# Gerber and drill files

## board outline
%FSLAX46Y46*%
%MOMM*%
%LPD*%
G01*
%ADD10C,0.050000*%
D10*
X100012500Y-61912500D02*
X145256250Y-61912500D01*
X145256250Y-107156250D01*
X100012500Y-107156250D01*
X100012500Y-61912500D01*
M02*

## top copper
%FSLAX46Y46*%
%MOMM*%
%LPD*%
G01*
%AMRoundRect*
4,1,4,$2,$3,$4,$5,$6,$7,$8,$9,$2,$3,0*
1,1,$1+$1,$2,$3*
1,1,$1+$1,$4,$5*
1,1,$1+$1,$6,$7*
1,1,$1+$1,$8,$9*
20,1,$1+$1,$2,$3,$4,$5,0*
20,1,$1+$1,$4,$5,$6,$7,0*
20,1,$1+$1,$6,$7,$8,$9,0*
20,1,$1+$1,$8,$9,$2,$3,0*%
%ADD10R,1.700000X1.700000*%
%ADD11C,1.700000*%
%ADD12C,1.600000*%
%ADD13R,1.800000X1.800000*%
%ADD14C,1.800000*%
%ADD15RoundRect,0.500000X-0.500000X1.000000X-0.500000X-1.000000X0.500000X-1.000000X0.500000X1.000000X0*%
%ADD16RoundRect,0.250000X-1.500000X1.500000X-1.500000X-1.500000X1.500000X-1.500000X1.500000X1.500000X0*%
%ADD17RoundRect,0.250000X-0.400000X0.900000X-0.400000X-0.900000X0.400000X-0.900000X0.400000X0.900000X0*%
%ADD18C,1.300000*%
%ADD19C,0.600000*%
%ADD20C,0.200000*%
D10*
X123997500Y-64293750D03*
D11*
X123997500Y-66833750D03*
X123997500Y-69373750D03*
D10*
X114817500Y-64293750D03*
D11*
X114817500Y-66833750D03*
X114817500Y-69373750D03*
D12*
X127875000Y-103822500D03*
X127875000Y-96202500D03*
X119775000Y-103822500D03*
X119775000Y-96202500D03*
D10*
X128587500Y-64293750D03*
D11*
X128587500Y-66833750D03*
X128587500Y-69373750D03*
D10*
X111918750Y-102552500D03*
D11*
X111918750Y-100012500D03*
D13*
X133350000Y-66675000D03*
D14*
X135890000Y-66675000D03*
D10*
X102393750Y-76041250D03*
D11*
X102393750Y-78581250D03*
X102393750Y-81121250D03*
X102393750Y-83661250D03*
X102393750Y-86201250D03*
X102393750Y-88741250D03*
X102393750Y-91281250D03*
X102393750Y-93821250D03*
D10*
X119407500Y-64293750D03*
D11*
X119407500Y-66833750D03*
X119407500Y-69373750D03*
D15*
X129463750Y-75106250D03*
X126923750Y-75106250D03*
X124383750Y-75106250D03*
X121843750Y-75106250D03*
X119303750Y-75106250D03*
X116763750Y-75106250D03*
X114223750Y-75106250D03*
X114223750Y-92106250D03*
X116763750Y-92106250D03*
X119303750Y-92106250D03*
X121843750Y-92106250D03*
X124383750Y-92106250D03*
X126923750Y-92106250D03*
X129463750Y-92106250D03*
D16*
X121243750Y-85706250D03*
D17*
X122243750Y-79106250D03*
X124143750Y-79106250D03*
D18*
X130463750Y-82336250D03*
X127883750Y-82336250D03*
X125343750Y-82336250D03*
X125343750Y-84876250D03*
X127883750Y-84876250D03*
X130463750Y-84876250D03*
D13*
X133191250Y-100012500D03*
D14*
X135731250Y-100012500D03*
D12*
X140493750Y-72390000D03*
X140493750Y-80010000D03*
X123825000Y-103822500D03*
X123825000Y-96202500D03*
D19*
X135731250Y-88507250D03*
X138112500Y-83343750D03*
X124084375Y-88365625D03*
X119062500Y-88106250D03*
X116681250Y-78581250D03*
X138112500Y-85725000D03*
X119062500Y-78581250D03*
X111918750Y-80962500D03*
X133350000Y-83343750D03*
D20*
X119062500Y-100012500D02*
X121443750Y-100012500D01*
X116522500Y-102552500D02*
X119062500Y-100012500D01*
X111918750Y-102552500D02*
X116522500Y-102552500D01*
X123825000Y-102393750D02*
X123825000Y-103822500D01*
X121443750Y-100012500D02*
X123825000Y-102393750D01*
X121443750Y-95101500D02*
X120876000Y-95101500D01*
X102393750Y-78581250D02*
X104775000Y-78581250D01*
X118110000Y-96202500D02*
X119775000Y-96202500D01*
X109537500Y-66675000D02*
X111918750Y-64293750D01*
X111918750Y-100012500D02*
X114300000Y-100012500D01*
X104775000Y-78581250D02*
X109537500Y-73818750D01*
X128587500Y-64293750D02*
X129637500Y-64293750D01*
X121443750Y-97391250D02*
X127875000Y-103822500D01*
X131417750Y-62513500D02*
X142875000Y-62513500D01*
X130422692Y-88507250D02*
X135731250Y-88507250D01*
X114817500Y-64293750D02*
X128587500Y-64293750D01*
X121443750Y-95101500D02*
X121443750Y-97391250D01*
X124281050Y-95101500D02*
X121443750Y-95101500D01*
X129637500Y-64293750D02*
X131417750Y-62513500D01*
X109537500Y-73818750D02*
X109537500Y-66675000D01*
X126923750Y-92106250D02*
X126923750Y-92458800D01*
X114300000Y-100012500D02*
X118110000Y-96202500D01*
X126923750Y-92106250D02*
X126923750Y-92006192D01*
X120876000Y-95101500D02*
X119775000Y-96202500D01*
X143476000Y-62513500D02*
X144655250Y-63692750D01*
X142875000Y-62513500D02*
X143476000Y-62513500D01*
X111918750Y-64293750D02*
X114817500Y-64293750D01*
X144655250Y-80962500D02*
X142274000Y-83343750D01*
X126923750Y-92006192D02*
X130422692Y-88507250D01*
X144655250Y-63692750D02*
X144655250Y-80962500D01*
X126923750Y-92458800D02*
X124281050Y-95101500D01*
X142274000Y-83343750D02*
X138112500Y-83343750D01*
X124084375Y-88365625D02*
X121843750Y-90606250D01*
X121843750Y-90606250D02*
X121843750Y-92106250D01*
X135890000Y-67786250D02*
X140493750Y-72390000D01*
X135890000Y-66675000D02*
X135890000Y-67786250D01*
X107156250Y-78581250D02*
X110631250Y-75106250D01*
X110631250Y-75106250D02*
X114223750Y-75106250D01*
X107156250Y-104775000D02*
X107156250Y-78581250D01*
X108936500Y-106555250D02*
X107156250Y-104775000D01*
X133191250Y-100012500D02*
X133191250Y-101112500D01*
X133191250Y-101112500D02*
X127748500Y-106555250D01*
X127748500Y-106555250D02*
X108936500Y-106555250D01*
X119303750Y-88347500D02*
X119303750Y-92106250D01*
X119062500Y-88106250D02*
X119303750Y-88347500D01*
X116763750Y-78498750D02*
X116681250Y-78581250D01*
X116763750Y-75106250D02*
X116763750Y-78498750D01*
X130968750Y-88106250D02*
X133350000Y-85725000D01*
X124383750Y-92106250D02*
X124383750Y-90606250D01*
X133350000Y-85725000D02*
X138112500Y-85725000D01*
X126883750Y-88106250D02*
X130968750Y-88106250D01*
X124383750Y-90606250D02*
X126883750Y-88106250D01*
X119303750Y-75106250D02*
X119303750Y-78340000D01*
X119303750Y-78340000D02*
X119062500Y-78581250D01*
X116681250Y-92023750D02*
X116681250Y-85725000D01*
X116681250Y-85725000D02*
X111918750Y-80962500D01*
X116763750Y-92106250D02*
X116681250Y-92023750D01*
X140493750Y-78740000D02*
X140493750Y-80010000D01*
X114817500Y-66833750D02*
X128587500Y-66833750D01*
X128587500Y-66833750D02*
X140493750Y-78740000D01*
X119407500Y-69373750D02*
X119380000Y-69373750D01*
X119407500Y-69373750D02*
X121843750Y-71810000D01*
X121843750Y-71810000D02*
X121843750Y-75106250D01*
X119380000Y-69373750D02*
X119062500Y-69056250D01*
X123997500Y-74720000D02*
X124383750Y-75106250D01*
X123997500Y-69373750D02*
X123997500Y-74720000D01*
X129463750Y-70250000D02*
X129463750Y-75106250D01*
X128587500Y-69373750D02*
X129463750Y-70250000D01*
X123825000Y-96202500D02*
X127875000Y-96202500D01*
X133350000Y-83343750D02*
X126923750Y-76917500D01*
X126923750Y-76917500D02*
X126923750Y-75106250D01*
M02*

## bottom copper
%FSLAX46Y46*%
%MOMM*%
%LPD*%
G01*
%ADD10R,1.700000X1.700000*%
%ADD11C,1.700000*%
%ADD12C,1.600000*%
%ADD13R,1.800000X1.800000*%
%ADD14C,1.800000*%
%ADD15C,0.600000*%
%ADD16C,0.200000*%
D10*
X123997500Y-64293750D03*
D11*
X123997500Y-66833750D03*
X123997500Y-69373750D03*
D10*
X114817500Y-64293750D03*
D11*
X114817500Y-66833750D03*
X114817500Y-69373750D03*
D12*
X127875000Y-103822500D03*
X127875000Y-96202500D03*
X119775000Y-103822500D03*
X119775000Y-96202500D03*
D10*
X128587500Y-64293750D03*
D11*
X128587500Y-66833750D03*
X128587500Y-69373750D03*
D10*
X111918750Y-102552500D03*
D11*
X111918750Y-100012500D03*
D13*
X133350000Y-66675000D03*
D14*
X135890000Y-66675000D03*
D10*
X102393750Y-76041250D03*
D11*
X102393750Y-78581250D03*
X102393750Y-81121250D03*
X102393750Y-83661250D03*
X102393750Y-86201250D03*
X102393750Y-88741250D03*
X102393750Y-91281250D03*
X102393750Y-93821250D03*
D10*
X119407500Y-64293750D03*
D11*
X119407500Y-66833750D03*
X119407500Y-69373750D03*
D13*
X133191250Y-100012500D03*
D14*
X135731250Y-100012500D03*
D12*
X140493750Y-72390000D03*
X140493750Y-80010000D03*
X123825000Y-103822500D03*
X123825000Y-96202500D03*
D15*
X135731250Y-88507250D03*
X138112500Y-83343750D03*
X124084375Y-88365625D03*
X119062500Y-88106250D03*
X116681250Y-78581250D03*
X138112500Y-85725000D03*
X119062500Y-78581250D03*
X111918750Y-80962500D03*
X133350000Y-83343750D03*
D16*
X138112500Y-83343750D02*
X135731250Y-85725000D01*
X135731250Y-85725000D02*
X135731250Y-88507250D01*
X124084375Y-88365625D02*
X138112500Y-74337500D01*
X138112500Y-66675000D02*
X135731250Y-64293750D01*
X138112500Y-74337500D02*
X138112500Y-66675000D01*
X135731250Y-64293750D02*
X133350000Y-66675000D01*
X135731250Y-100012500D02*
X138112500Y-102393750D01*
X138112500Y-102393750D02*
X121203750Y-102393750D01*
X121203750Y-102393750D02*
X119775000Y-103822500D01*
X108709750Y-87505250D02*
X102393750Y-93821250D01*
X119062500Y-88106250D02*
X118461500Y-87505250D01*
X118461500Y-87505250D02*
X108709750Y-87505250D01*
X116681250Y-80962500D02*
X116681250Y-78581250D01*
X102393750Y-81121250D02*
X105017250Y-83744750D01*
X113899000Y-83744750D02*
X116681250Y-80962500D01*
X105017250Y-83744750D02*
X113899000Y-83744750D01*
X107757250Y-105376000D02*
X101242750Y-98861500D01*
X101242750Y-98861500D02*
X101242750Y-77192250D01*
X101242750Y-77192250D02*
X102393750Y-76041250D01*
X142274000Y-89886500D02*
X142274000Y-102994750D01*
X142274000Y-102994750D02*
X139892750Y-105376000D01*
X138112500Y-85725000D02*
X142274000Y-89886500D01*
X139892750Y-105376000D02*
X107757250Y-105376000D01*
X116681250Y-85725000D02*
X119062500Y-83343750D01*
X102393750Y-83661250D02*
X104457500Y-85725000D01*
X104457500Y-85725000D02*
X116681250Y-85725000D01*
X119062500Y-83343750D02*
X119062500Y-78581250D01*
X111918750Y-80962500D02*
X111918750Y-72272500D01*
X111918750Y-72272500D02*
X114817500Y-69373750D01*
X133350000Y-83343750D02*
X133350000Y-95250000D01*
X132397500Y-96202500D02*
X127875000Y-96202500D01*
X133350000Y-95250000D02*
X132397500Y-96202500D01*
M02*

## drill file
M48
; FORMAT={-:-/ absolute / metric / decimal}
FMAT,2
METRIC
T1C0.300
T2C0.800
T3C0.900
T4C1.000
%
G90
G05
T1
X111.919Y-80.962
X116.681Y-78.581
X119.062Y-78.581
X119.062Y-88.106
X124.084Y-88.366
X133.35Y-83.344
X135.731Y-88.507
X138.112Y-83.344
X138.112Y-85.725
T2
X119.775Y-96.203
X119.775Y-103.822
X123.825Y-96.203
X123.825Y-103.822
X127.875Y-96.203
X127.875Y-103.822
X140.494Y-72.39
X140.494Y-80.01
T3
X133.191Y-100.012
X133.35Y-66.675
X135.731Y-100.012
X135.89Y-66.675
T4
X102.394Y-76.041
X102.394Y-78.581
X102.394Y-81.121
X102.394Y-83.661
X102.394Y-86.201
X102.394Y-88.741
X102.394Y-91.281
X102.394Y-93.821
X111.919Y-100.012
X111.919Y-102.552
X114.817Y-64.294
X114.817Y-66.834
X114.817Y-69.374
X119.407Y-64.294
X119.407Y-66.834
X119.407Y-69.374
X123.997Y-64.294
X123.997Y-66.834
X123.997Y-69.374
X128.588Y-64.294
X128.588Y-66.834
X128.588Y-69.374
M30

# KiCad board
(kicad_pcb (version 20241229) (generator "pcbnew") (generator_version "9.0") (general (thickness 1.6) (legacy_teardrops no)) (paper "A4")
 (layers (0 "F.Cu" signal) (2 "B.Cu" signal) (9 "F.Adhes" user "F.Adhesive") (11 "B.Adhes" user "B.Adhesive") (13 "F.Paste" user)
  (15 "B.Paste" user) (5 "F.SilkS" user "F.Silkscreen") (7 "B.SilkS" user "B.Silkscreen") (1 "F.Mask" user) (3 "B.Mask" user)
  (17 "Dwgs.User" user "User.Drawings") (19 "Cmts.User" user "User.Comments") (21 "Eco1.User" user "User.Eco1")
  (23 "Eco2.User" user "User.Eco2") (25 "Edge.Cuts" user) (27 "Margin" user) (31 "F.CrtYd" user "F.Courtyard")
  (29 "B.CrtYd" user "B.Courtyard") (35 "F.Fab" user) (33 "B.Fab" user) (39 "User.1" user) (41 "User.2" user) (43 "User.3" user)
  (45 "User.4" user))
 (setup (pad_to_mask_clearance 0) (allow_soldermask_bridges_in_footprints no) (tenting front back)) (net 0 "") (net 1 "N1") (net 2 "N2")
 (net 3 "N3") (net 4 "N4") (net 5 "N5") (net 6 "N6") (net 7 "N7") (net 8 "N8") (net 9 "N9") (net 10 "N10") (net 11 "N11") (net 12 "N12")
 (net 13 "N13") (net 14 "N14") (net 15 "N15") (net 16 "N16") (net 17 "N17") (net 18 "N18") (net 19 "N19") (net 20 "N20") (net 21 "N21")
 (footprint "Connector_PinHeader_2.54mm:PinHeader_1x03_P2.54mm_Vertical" (layer "F.Cu") (at 123.9975 64.29375)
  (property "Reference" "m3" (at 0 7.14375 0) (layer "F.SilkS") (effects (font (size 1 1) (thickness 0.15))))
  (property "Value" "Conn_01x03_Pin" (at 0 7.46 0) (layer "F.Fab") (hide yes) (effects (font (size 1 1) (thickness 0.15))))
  (pad "1" thru_hole rect (at 0 0) (size 1.7 1.7) (drill 1) (layers "*.Cu" "*.Mask") (remove_unused_layers no) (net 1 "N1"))
  (pad "2" thru_hole circle (at 0 2.54) (size 1.7 1.7) (drill 1) (layers "*.Cu" "*.Mask") (remove_unused_layers no) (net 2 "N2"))
  (pad "3" thru_hole circle (at 0 5.08) (size 1.7 1.7) (drill 1) (layers "*.Cu" "*.Mask") (remove_unused_layers no) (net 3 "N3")))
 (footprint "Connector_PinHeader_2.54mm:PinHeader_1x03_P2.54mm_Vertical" (layer "F.Cu") (at 114.8175 64.29375)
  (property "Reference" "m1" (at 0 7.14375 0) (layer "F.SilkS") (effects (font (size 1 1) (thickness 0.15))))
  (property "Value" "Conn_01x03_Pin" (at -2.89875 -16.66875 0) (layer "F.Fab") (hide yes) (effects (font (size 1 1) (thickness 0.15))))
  (pad "1" thru_hole rect (at 0 0) (size 1.7 1.7) (drill 1) (layers "*.Cu" "*.Mask") (remove_unused_layers no) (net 1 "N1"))
  (pad "2" thru_hole circle (at 0 2.54) (size 1.7 1.7) (drill 1) (layers "*.Cu" "*.Mask") (remove_unused_layers no) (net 2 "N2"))
  (pad "3" thru_hole circle (at 0 5.08) (size 1.7 1.7) (drill 1) (layers "*.Cu" "*.Mask") (remove_unused_layers no) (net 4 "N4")))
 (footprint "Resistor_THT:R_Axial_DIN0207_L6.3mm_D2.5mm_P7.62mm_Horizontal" (layer "F.Cu") (at 127.875 103.8225 90)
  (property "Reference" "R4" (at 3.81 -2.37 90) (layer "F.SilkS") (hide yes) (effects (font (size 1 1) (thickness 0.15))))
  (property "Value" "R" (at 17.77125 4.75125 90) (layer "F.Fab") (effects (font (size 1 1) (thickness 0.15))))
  (pad "1" thru_hole circle (at 0 0 90) (size 1.6 1.6) (drill 0.8) (layers "*.Cu" "*.Mask") (remove_unused_layers no) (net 1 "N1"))
  (pad "2" thru_hole circle (at 7.62 0 90) (size 1.6 1.6) (drill 0.8) (layers "*.Cu" "*.Mask") (remove_unused_layers no) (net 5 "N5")))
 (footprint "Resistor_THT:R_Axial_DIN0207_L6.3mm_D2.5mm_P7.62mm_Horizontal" (layer "F.Cu") (at 119.775 103.8225 90)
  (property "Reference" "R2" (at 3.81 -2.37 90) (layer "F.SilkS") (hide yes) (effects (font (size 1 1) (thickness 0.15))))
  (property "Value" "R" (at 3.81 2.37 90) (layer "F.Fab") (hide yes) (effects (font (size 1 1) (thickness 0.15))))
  (pad "1" thru_hole circle (at 0 0 90) (size 1.6 1.6) (drill 0.8) (layers "*.Cu" "*.Mask") (remove_unused_layers no) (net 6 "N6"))
  (pad "2" thru_hole circle (at 7.62 0 90) (size 1.6 1.6) (drill 0.8) (layers "*.Cu" "*.Mask") (remove_unused_layers no) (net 1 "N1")))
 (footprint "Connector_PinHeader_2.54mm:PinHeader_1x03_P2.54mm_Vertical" (layer "F.Cu") (at 128.5875 64.29375)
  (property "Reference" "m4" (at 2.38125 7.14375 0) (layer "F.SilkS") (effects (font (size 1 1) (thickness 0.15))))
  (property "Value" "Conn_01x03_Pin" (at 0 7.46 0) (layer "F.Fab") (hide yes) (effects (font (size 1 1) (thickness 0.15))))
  (pad "1" thru_hole rect (at 0 0) (size 1.7 1.7) (drill 1) (layers "*.Cu" "*.Mask") (remove_unused_layers no) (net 1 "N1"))
  (pad "2" thru_hole circle (at 0 2.54) (size 1.7 1.7) (drill 1) (layers "*.Cu" "*.Mask") (remove_unused_layers no) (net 2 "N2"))
  (pad "3" thru_hole circle (at 0 5.08) (size 1.7 1.7) (drill 1) (layers "*.Cu" "*.Mask") (remove_unused_layers no) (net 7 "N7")))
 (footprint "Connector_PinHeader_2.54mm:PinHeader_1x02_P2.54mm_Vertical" (layer "F.Cu") (at 111.91875 102.5525 180)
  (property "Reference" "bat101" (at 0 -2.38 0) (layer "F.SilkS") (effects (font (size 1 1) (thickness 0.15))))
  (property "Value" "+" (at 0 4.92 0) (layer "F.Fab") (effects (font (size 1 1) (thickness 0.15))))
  (pad "1" thru_hole rect (at 0 0 180) (size 1.7 1.7) (drill 1) (layers "*.Cu" "*.Mask") (remove_unused_layers no) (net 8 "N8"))
  (pad "2" thru_hole circle (at 0 2.54 180) (size 1.7 1.7) (drill 1) (layers "*.Cu" "*.Mask") (remove_unused_layers no) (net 1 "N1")))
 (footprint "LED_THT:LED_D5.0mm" (layer "F.Cu") (at 133.35 66.675)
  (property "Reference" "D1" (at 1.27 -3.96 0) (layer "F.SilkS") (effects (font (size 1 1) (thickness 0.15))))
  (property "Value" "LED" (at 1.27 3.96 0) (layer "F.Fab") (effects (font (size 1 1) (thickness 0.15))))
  (pad "1" thru_hole rect (at 0 0) (size 1.8 1.8) (drill 0.9) (layers "*.Cu" "*.Mask") (remove_unused_layers no) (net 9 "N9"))
  (pad "2" thru_hole circle (at 2.54 0) (size 1.8 1.8) (drill 0.9) (layers "*.Cu" "*.Mask") (remove_unused_layers no) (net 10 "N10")))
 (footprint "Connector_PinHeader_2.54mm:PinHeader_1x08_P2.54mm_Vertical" (layer "F.Cu") (at 102.39375 76.04125)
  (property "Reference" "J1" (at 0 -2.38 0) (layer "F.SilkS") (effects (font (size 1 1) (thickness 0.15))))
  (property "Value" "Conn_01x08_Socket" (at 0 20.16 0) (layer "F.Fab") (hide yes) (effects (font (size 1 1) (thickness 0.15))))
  (pad "1" thru_hole rect (at 0 0) (size 1.7 1.7) (drill 1) (layers "*.Cu" "*.Mask") (remove_unused_layers no) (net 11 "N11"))
  (pad "2" thru_hole circle (at 0 2.54) (size 1.7 1.7) (drill 1) (layers "*.Cu" "*.Mask") (remove_unused_layers no) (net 1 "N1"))
  (pad "3" thru_hole circle (at 0 5.08) (size 1.7 1.7) (drill 1) (layers "*.Cu" "*.Mask") (remove_unused_layers no) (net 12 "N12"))
  (pad "4" thru_hole circle (at 0 7.62) (size 1.7 1.7) (drill 1) (layers "*.Cu" "*.Mask") (remove_unused_layers no) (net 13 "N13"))
  (pad "5" thru_hole circle (at 0 10.16) (size 1.7 1.7) (drill 1) (layers "*.Cu" "*.Mask") (remove_unused_layers no) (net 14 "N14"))
  (pad "6" thru_hole circle (at 0 12.7) (size 1.7 1.7) (drill 1) (layers "*.Cu" "*.Mask") (remove_unused_layers no) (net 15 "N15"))
  (pad "7" thru_hole circle (at 0 15.24) (size 1.7 1.7) (drill 1) (layers "*.Cu" "*.Mask") (remove_unused_layers no) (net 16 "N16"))
  (pad "8" thru_hole circle (at 0 17.78) (size 1.7 1.7) (drill 1) (layers "*.Cu" "*.Mask") (remove_unused_layers no) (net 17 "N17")))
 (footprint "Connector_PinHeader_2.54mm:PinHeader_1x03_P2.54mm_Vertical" (layer "F.Cu") (at 119.4075 64.29375)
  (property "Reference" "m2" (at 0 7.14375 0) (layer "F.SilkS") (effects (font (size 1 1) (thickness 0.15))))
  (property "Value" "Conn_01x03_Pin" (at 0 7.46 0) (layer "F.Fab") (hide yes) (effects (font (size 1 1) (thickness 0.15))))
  (pad "1" thru_hole rect (at 0 0) (size 1.7 1.7) (drill 1) (layers "*.Cu" "*.Mask") (remove_unused_layers no) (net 1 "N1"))
  (pad "2" thru_hole circle (at 0 2.54) (size 1.7 1.7) (drill 1) (layers "*.Cu" "*.Mask") (remove_unused_layers no) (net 2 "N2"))
  (pad "3" thru_hole circle (at 0 5.08) (size 1.7 1.7) (drill 1) (layers "*.Cu" "*.Mask") (remove_unused_layers no) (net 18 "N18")))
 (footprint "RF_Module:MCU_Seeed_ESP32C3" (layer "F.Cu") (at 121.84375 83.60625 -90)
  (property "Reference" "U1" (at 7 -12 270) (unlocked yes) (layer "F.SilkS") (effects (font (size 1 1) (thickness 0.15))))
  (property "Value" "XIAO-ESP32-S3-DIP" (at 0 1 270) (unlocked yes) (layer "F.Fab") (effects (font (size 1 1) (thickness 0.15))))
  (pad "" smd roundrect (at 1.1 -0.4 270) (size 1.5 1.5) (layers "F.Paste") (roundrect_rratio 0.1666666667))
  (pad "" smd roundrect (at 1.1 1.6 270) (size 1.5 1.5) (layers "F.Paste") (roundrect_rratio 0.1666666667))
  (pad "" smd roundrect (at 3.1 -0.4 270) (size 1.5 1.5) (layers "F.Paste") (roundrect_rratio 0.1666666667))
  (pad "" smd roundrect (at 3.1 1.6 270) (size 1.5 1.5) (layers "F.Paste") (roundrect_rratio 0.1666666667))
  (pad "1" smd roundrect (at -8.5 -7.62 270) (size 3 2) (layers "F.Cu" "F.Mask" "F.Paste") (roundrect_rratio 0.25) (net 7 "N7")
   (thermal_bridge_angle 45))
  (pad "2" smd roundrect (at -8.5 -5.08 270) (size 3 2) (layers "F.Cu" "F.Mask" "F.Paste") (roundrect_rratio 0.25) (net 5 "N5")
   (thermal_bridge_angle 45))
  (pad "3" smd roundrect (at -8.5 -2.54 270) (size 3 2) (layers "F.Cu" "F.Mask" "F.Paste") (roundrect_rratio 0.25) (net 3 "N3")
   (thermal_bridge_angle 45))
  (pad "4" smd roundrect (at -8.5 0 270) (size 3 2) (layers "F.Cu" "F.Mask" "F.Paste") (roundrect_rratio 0.25) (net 18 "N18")
   (thermal_bridge_angle 45))
  (pad "5" smd roundrect (at -8.5 2.54 270) (size 3 2) (layers "F.Cu" "F.Mask" "F.Paste") (roundrect_rratio 0.25) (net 13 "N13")
   (thermal_bridge_angle 45))
  (pad "6" smd roundrect (at -8.5 5.08 270) (size 3 2) (layers "F.Cu" "F.Mask" "F.Paste") (roundrect_rratio 0.25) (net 12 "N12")
   (thermal_bridge_angle 45))
  (pad "7" smd roundrect (at -8.5 7.62 270) (size 3 2) (layers "F.Cu" "F.Mask" "F.Paste") (roundrect_rratio 0.25) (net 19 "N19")
   (thermal_bridge_angle 45))
  (pad "8" smd roundrect (at 8.5 7.62 270) (size 3 2) (layers "F.Cu" "F.Mask" "F.Paste") (roundrect_rratio 0.25) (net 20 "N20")
   (thermal_bridge_angle 45))
  (pad "9" smd roundrect (at 8.5 5.08 270) (size 3 2) (layers "F.Cu" "F.Mask" "F.Paste") (roundrect_rratio 0.25) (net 4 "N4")
   (thermal_bridge_angle 45))
  (pad "10" smd roundrect (at 8.5 2.54 270) (size 3 2) (layers "F.Cu" "F.Mask" "F.Paste") (roundrect_rratio 0.25) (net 17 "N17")
   (thermal_bridge_angle 45))
  (pad "11" smd roundrect (at 8.5 0 270) (size 3 2) (layers "F.Cu" "F.Mask" "F.Paste") (roundrect_rratio 0.25) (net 9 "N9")
   (thermal_bridge_angle 45))
  (pad "12" smd roundrect (at 8.5 -2.54 270) (size 3 2) (layers "F.Cu" "F.Mask" "F.Paste") (roundrect_rratio 0.25) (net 11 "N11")
   (thermal_bridge_angle 45))
  (pad "13" smd roundrect (at 8.5 -5.08 270) (size 3 2) (layers "F.Cu" "F.Mask" "F.Paste") (roundrect_rratio 0.25) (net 1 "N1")
   (thermal_bridge_angle 45))
  (pad "14" smd roundrect (at 8.5 -7.62 270) (size 3 2) (layers "F.Cu" "F.Mask" "F.Paste") (roundrect_rratio 0.25) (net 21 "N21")
   (thermal_bridge_angle 45))
  (pad "15" smd roundrect (at 2.1 0.6 270) (size 3.5 3.5) (layers "F.Cu" "F.Mask") (roundrect_rratio 0.07142857143))
  (pad "16" smd roundrect (at -4.5 -0.4 270) (size 2.3 1.3) (layers "F.Cu" "F.Mask" "F.Paste") (roundrect_rratio 0.1923076923))
  (pad "17" smd roundrect (at -4.5 -2.3 270) (size 2.3 1.3) (layers "F.Cu" "F.Mask" "F.Paste") (roundrect_rratio 0.1923076923))
  (pad "18" smd circle (at -1.27 -8.62 270) (size 1.3 1.3) (layers "F.Cu" "F.Mask" "F.Paste"))
  (pad "19" smd circle (at -1.27 -6.04 270) (size 1.3 1.3) (layers "F.Cu" "F.Mask" "F.Paste"))
  (pad "20" smd circle (at -1.27 -3.5 270) (size 1.3 1.3) (layers "F.Cu" "F.Mask" "F.Paste"))
  (pad "21" smd circle (at 1.27 -3.5 270) (size 1.3 1.3) (layers "F.Cu" "F.Mask" "F.Paste"))
  (pad "22" smd circle (at 1.27 -6.04 270) (size 1.3 1.3) (layers "F.Cu" "F.Mask" "F.Paste"))
  (pad "23" smd circle (at 1.27 -8.62 270) (size 1.3 1.3) (layers "F.Cu" "F.Mask" "F.Paste")))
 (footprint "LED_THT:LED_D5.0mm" (layer "F.Cu") (at 133.19125 100.0125)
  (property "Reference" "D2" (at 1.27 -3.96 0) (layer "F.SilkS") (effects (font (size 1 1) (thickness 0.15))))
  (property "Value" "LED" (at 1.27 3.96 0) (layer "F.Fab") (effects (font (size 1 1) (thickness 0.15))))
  (pad "1" thru_hole rect (at 0 0) (size 1.8 1.8) (drill 0.9) (layers "*.Cu" "*.Mask") (remove_unused_layers no) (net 19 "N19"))
  (pad "2" thru_hole circle (at 2.54 0) (size 1.8 1.8) (drill 0.9) (layers "*.Cu" "*.Mask") (remove_unused_layers no) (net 6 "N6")))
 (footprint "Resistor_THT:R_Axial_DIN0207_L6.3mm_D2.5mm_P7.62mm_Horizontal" (layer "F.Cu") (at 140.49375 72.39 -90)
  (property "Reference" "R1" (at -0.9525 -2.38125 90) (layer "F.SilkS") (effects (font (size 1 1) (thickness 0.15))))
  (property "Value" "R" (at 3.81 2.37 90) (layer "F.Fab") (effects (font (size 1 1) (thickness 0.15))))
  (pad "1" thru_hole circle (at 0 0 270) (size 1.6 1.6) (drill 0.8) (layers "*.Cu" "*.Mask") (remove_unused_layers no) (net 10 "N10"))
  (pad "2" thru_hole circle (at 7.62 0 270) (size 1.6 1.6) (drill 0.8) (layers "*.Cu" "*.Mask") (remove_unused_layers no) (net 2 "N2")))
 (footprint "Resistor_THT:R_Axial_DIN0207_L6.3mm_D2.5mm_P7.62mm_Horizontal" (layer "F.Cu") (at 123.825 103.8225 90)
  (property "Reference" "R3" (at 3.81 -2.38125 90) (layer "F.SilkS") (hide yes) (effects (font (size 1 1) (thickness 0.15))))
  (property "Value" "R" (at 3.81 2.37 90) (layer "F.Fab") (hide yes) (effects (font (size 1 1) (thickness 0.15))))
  (pad "1" thru_hole circle (at 0 0 90) (size 1.6 1.6) (drill 0.8) (layers "*.Cu" "*.Mask") (remove_unused_layers no) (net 8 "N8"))
  (pad "2" thru_hole circle (at 7.62 0 90) (size 1.6 1.6) (drill 0.8) (layers "*.Cu" "*.Mask") (remove_unused_layers no) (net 5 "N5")))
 (gr_rect (start 100.0125 61.9125) (end 145.25625 107.15625) (stroke (width 0.05) (type default)) (fill no) (layer "Edge.Cuts"))
 (segment (start 119.0625 100.0125) (end 121.44375 100.0125) (width 0.2) (layer "F.Cu") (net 8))
 (segment (start 116.5225 102.5525) (end 119.0625 100.0125) (width 0.2) (layer "F.Cu") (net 8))
 (segment (start 111.91875 102.5525) (end 116.5225 102.5525) (width 0.2) (layer "F.Cu") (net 8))
 (segment (start 123.825 102.39375) (end 123.825 103.8225) (width 0.2) (layer "F.Cu") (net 8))
 (segment (start 121.44375 100.0125) (end 123.825 102.39375) (width 0.2) (layer "F.Cu") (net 8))
 (segment (start 121.44375 95.1015) (end 120.876 95.1015) (width 0.2) (layer "F.Cu") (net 1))
 (segment (start 102.39375 78.58125) (end 104.775 78.58125) (width 0.2) (layer "F.Cu") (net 1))
 (segment (start 118.11 96.2025) (end 119.775 96.2025) (width 0.2) (layer "F.Cu") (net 1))
 (segment (start 109.5375 66.675) (end 111.91875 64.29375) (width 0.2) (layer "F.Cu") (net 1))
 (segment (start 111.91875 100.0125) (end 114.3 100.0125) (width 0.2) (layer "F.Cu") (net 1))
 (segment (start 104.775 78.58125) (end 109.5375 73.81875) (width 0.2) (layer "F.Cu") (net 1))
 (segment (start 128.5875 64.29375) (end 129.6375 64.29375) (width 0.2) (layer "F.Cu") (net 1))
 (segment (start 121.44375 97.39125) (end 127.875 103.8225) (width 0.2) (layer "F.Cu") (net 1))
 (segment (start 131.41775 62.5135) (end 142.875 62.5135) (width 0.2) (layer "F.Cu") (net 1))
 (segment (start 130.422692 88.50725) (end 135.73125 88.50725) (width 0.2) (layer "F.Cu") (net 1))
 (segment (start 114.8175 64.29375) (end 128.5875 64.29375) (width 0.2) (layer "F.Cu") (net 1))
 (segment (start 121.44375 95.1015) (end 121.44375 97.39125) (width 0.2) (layer "F.Cu") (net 1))
 (segment (start 124.28105 95.1015) (end 121.44375 95.1015) (width 0.2) (layer "F.Cu") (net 1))
 (segment (start 129.6375 64.29375) (end 131.41775 62.5135) (width 0.2) (layer "F.Cu") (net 1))
 (segment (start 109.5375 73.81875) (end 109.5375 66.675) (width 0.2) (layer "F.Cu") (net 1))
 (segment (start 126.92375 92.10625) (end 126.92375 92.4588) (width 0.2) (layer "F.Cu") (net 1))
 (segment (start 114.3 100.0125) (end 118.11 96.2025) (width 0.2) (layer "F.Cu") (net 1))
 (segment (start 126.92375 92.10625) (end 126.92375 92.006192) (width 0.2) (layer "F.Cu") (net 1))
 (segment (start 120.876 95.1015) (end 119.775 96.2025) (width 0.2) (layer "F.Cu") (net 1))
 (segment (start 143.476 62.5135) (end 144.65525 63.69275) (width 0.2) (layer "F.Cu") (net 1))
 (segment (start 142.875 62.5135) (end 143.476 62.5135) (width 0.2) (layer "F.Cu") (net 1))
 (segment (start 111.91875 64.29375) (end 114.8175 64.29375) (width 0.2) (layer "F.Cu") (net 1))
 (segment (start 144.65525 80.9625) (end 142.274 83.34375) (width 0.2) (layer "F.Cu") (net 1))
 (segment (start 126.92375 92.006192) (end 130.422692 88.50725) (width 0.2) (layer "F.Cu") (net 1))
 (segment (start 144.65525 63.69275) (end 144.65525 80.9625) (width 0.2) (layer "F.Cu") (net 1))
 (segment (start 126.92375 92.4588) (end 124.28105 95.1015) (width 0.2) (layer "F.Cu") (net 1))
 (segment (start 142.274 83.34375) (end 138.1125 83.34375) (width 0.2) (layer "F.Cu") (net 1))
 (via (at 135.73125 88.50725) (size 0.6) (drill 0.3) (layers "F.Cu" "B.Cu") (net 1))
 (via (at 138.1125 83.34375) (size 0.6) (drill 0.3) (layers "F.Cu" "B.Cu") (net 1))
 (segment (start 138.1125 83.34375) (end 135.73125 85.725) (width 0.2) (layer "B.Cu") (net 1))
 (segment (start 135.73125 85.725) (end 135.73125 88.50725) (width 0.2) (layer "B.Cu") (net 1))
 (segment (start 124.084375 88.365625) (end 121.84375 90.60625) (width 0.2) (layer "F.Cu") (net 9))
 (segment (start 121.84375 90.60625) (end 121.84375 92.10625) (width 0.2) (layer "F.Cu") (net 9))
 (via (at 124.084375 88.365625) (size 0.6) (drill 0.3) (layers "F.Cu" "B.Cu") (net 9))
 (segment (start 124.084375 88.365625) (end 138.1125 74.3375) (width 0.2) (layer "B.Cu") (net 9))
 (segment (start 138.1125 66.675) (end 135.73125 64.29375) (width 0.2) (layer "B.Cu") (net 9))
 (segment (start 138.1125 74.3375) (end 138.1125 66.675) (width 0.2) (layer "B.Cu") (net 9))
 (segment (start 135.73125 64.29375) (end 133.35 66.675) (width 0.2) (layer "B.Cu") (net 9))
 (segment (start 135.89 67.78625) (end 140.49375 72.39) (width 0.2) (layer "F.Cu") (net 10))
 (segment (start 135.89 66.675) (end 135.89 67.78625) (width 0.2) (layer "F.Cu") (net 10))
 (segment (start 107.15625 78.58125) (end 110.63125 75.10625) (width 0.2) (layer "F.Cu") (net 19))
 (segment (start 110.63125 75.10625) (end 114.22375 75.10625) (width 0.2) (layer "F.Cu") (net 19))
 (segment (start 107.15625 104.775) (end 107.15625 78.58125) (width 0.2) (layer "F.Cu") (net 19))
 (segment (start 108.9365 106.55525) (end 107.15625 104.775) (width 0.2) (layer "F.Cu") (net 19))
 (segment (start 133.19125 100.0125) (end 133.19125 101.1125) (width 0.2) (layer "F.Cu") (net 19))
 (segment (start 133.19125 101.1125) (end 127.7485 106.55525) (width 0.2) (layer "F.Cu") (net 19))
 (segment (start 127.7485 106.55525) (end 108.9365 106.55525) (width 0.2) (layer "F.Cu") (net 19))
 (segment (start 135.73125 100.0125) (end 138.1125 102.39375) (width 0.2) (layer "B.Cu") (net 6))
 (segment (start 138.1125 102.39375) (end 121.20375 102.39375) (width 0.2) (layer "B.Cu") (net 6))
 (segment (start 121.20375 102.39375) (end 119.775 103.8225) (width 0.2) (layer "B.Cu") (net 6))
 (segment (start 119.30375 88.3475) (end 119.30375 92.10625) (width 0.2) (layer "F.Cu") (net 17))
 (segment (start 119.0625 88.10625) (end 119.30375 88.3475) (width 0.2) (layer "F.Cu") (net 17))
 (via (at 119.0625 88.10625) (size 0.6) (drill 0.3) (layers "F.Cu" "B.Cu") (free yes) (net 17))
 (segment (start 108.70975 87.50525) (end 102.39375 93.82125) (width 0.2) (layer "B.Cu") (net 17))
 (segment (start 119.0625 88.10625) (end 118.4615 87.50525) (width 0.2) (layer "B.Cu") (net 17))
 (segment (start 118.4615 87.50525) (end 108.70975 87.50525) (width 0.2) (layer "B.Cu") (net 17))
 (segment (start 116.76375 78.49875) (end 116.68125 78.58125) (width 0.2) (layer "F.Cu") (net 12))
 (segment (start 116.76375 75.10625) (end 116.76375 78.49875) (width 0.2) (layer "F.Cu") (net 12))
 (via (at 116.68125 78.58125) (size 0.6) (drill 0.3) (layers "F.Cu" "B.Cu") (free yes) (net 12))
 (segment (start 116.68125 80.9625) (end 116.68125 78.58125) (width 0.2) (layer "B.Cu") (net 12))
 (segment (start 102.39375 81.12125) (end 105.01725 83.74475) (width 0.2) (layer "B.Cu") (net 12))
 (segment (start 113.899 83.74475) (end 116.68125 80.9625) (width 0.2) (layer "B.Cu") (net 12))
 (segment (start 105.01725 83.74475) (end 113.899 83.74475) (width 0.2) (layer "B.Cu") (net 12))
 (segment (start 130.96875 88.10625) (end 133.35 85.725) (width 0.2) (layer "F.Cu") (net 11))
 (segment (start 124.38375 92.10625) (end 124.38375 90.60625) (width 0.2) (layer "F.Cu") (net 11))
 (segment (start 133.35 85.725) (end 138.1125 85.725) (width 0.2) (layer "F.Cu") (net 11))
 (segment (start 126.88375 88.10625) (end 130.96875 88.10625) (width 0.2) (layer "F.Cu") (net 11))
 (segment (start 124.38375 90.60625) (end 126.88375 88.10625) (width 0.2) (layer "F.Cu") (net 11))
 (via (at 138.1125 85.725) (size 0.6) (drill 0.3) (layers "F.Cu" "B.Cu") (free yes) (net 11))
 (segment (start 107.75725 105.376) (end 101.24275 98.8615) (width 0.2) (layer "B.Cu") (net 11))
 (segment (start 101.24275 98.8615) (end 101.24275 77.19225) (width 0.2) (layer "B.Cu") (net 11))
 (segment (start 101.24275 77.19225) (end 102.39375 76.04125) (width 0.2) (layer "B.Cu") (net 11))
 (segment (start 142.274 89.8865) (end 142.274 102.99475) (width 0.2) (layer "B.Cu") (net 11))
 (segment (start 142.274 102.99475) (end 139.89275 105.376) (width 0.2) (layer "B.Cu") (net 11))
 (segment (start 138.1125 85.725) (end 142.274 89.8865) (width 0.2) (layer "B.Cu") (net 11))
 (segment (start 139.89275 105.376) (end 107.75725 105.376) (width 0.2) (layer "B.Cu") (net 11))
 (segment (start 119.30375 75.10625) (end 119.30375 78.34) (width 0.2) (layer "F.Cu") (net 13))
 (segment (start 119.30375 78.34) (end 119.0625 78.58125) (width 0.2) (layer "F.Cu") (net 13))
 (via (at 119.0625 78.58125) (size 0.6) (drill 0.3) (layers "F.Cu" "B.Cu") (free yes) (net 13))
 (segment (start 116.68125 85.725) (end 119.0625 83.34375) (width 0.2) (layer "B.Cu") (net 13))
 (segment (start 102.39375 83.66125) (end 104.4575 85.725) (width 0.2) (layer "B.Cu") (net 13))
 (segment (start 104.4575 85.725) (end 116.68125 85.725) (width 0.2) (layer "B.Cu") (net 13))
 (segment (start 119.0625 83.34375) (end 119.0625 78.58125) (width 0.2) (layer "B.Cu") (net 13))
 (segment (start 116.68125 92.02375) (end 116.68125 85.725) (width 0.2) (layer "F.Cu") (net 4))
 (segment (start 116.68125 85.725) (end 111.91875 80.9625) (width 0.2) (layer "F.Cu") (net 4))
 (segment (start 116.76375 92.10625) (end 116.68125 92.02375) (width 0.2) (layer "F.Cu") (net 4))
 (via (at 111.91875 80.9625) (size 0.6) (drill 0.3) (layers "F.Cu" "B.Cu") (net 4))
 (segment (start 111.91875 80.9625) (end 111.91875 72.2725) (width 0.2) (layer "B.Cu") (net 4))
 (segment (start 111.91875 72.2725) (end 114.8175 69.37375) (width 0.2) (layer "B.Cu") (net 4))
 (segment (start 140.49375 78.74) (end 140.49375 80.01) (width 0.2) (layer "F.Cu") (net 2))
 (segment (start 114.8175 66.83375) (end 128.5875 66.83375) (width 0.2) (layer "F.Cu") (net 2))
 (segment (start 128.5875 66.83375) (end 140.49375 78.74) (width 0.2) (layer "F.Cu") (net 2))
 (segment (start 119.4075 69.37375) (end 119.38 69.37375) (width 0.2) (layer "F.Cu") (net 18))
 (segment (start 119.4075 69.37375) (end 121.84375 71.81) (width 0.2) (layer "F.Cu") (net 18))
 (segment (start 121.84375 71.81) (end 121.84375 75.10625) (width 0.2) (layer "F.Cu") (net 18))
 (segment (start 119.38 69.37375) (end 119.0625 69.05625) (width 0.2) (layer "F.Cu") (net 18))
 (segment (start 123.9975 74.72) (end 124.38375 75.10625) (width 0.2) (layer "F.Cu") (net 3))
 (segment (start 123.9975 69.37375) (end 123.9975 74.72) (width 0.2) (layer "F.Cu") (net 3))
 (segment (start 129.46375 70.25) (end 129.46375 75.10625) (width 0.2) (layer "F.Cu") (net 7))
 (segment (start 128.5875 69.37375) (end 129.46375 70.25) (width 0.2) (layer "F.Cu") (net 7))
 (segment (start 123.825 96.2025) (end 127.875 96.2025) (width 0.2) (layer "F.Cu") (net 5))
 (segment (start 133.35 83.34375) (end 126.92375 76.9175) (width 0.2) (layer "F.Cu") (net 5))
 (segment (start 126.92375 76.9175) (end 126.92375 75.10625) (width 0.2) (layer "F.Cu") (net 5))
 (via (at 133.35 83.34375) (size 0.6) (drill 0.3) (layers "F.Cu" "B.Cu") (free yes) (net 5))
 (segment (start 133.35 83.34375) (end 133.35 95.25) (width 0.2) (layer "B.Cu") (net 5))
 (segment (start 132.3975 96.2025) (end 127.875 96.2025) (width 0.2) (layer "B.Cu") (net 5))
 (segment (start 133.35 95.25) (end 132.3975 96.2025) (width 0.2) (layer "B.Cu") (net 5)))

